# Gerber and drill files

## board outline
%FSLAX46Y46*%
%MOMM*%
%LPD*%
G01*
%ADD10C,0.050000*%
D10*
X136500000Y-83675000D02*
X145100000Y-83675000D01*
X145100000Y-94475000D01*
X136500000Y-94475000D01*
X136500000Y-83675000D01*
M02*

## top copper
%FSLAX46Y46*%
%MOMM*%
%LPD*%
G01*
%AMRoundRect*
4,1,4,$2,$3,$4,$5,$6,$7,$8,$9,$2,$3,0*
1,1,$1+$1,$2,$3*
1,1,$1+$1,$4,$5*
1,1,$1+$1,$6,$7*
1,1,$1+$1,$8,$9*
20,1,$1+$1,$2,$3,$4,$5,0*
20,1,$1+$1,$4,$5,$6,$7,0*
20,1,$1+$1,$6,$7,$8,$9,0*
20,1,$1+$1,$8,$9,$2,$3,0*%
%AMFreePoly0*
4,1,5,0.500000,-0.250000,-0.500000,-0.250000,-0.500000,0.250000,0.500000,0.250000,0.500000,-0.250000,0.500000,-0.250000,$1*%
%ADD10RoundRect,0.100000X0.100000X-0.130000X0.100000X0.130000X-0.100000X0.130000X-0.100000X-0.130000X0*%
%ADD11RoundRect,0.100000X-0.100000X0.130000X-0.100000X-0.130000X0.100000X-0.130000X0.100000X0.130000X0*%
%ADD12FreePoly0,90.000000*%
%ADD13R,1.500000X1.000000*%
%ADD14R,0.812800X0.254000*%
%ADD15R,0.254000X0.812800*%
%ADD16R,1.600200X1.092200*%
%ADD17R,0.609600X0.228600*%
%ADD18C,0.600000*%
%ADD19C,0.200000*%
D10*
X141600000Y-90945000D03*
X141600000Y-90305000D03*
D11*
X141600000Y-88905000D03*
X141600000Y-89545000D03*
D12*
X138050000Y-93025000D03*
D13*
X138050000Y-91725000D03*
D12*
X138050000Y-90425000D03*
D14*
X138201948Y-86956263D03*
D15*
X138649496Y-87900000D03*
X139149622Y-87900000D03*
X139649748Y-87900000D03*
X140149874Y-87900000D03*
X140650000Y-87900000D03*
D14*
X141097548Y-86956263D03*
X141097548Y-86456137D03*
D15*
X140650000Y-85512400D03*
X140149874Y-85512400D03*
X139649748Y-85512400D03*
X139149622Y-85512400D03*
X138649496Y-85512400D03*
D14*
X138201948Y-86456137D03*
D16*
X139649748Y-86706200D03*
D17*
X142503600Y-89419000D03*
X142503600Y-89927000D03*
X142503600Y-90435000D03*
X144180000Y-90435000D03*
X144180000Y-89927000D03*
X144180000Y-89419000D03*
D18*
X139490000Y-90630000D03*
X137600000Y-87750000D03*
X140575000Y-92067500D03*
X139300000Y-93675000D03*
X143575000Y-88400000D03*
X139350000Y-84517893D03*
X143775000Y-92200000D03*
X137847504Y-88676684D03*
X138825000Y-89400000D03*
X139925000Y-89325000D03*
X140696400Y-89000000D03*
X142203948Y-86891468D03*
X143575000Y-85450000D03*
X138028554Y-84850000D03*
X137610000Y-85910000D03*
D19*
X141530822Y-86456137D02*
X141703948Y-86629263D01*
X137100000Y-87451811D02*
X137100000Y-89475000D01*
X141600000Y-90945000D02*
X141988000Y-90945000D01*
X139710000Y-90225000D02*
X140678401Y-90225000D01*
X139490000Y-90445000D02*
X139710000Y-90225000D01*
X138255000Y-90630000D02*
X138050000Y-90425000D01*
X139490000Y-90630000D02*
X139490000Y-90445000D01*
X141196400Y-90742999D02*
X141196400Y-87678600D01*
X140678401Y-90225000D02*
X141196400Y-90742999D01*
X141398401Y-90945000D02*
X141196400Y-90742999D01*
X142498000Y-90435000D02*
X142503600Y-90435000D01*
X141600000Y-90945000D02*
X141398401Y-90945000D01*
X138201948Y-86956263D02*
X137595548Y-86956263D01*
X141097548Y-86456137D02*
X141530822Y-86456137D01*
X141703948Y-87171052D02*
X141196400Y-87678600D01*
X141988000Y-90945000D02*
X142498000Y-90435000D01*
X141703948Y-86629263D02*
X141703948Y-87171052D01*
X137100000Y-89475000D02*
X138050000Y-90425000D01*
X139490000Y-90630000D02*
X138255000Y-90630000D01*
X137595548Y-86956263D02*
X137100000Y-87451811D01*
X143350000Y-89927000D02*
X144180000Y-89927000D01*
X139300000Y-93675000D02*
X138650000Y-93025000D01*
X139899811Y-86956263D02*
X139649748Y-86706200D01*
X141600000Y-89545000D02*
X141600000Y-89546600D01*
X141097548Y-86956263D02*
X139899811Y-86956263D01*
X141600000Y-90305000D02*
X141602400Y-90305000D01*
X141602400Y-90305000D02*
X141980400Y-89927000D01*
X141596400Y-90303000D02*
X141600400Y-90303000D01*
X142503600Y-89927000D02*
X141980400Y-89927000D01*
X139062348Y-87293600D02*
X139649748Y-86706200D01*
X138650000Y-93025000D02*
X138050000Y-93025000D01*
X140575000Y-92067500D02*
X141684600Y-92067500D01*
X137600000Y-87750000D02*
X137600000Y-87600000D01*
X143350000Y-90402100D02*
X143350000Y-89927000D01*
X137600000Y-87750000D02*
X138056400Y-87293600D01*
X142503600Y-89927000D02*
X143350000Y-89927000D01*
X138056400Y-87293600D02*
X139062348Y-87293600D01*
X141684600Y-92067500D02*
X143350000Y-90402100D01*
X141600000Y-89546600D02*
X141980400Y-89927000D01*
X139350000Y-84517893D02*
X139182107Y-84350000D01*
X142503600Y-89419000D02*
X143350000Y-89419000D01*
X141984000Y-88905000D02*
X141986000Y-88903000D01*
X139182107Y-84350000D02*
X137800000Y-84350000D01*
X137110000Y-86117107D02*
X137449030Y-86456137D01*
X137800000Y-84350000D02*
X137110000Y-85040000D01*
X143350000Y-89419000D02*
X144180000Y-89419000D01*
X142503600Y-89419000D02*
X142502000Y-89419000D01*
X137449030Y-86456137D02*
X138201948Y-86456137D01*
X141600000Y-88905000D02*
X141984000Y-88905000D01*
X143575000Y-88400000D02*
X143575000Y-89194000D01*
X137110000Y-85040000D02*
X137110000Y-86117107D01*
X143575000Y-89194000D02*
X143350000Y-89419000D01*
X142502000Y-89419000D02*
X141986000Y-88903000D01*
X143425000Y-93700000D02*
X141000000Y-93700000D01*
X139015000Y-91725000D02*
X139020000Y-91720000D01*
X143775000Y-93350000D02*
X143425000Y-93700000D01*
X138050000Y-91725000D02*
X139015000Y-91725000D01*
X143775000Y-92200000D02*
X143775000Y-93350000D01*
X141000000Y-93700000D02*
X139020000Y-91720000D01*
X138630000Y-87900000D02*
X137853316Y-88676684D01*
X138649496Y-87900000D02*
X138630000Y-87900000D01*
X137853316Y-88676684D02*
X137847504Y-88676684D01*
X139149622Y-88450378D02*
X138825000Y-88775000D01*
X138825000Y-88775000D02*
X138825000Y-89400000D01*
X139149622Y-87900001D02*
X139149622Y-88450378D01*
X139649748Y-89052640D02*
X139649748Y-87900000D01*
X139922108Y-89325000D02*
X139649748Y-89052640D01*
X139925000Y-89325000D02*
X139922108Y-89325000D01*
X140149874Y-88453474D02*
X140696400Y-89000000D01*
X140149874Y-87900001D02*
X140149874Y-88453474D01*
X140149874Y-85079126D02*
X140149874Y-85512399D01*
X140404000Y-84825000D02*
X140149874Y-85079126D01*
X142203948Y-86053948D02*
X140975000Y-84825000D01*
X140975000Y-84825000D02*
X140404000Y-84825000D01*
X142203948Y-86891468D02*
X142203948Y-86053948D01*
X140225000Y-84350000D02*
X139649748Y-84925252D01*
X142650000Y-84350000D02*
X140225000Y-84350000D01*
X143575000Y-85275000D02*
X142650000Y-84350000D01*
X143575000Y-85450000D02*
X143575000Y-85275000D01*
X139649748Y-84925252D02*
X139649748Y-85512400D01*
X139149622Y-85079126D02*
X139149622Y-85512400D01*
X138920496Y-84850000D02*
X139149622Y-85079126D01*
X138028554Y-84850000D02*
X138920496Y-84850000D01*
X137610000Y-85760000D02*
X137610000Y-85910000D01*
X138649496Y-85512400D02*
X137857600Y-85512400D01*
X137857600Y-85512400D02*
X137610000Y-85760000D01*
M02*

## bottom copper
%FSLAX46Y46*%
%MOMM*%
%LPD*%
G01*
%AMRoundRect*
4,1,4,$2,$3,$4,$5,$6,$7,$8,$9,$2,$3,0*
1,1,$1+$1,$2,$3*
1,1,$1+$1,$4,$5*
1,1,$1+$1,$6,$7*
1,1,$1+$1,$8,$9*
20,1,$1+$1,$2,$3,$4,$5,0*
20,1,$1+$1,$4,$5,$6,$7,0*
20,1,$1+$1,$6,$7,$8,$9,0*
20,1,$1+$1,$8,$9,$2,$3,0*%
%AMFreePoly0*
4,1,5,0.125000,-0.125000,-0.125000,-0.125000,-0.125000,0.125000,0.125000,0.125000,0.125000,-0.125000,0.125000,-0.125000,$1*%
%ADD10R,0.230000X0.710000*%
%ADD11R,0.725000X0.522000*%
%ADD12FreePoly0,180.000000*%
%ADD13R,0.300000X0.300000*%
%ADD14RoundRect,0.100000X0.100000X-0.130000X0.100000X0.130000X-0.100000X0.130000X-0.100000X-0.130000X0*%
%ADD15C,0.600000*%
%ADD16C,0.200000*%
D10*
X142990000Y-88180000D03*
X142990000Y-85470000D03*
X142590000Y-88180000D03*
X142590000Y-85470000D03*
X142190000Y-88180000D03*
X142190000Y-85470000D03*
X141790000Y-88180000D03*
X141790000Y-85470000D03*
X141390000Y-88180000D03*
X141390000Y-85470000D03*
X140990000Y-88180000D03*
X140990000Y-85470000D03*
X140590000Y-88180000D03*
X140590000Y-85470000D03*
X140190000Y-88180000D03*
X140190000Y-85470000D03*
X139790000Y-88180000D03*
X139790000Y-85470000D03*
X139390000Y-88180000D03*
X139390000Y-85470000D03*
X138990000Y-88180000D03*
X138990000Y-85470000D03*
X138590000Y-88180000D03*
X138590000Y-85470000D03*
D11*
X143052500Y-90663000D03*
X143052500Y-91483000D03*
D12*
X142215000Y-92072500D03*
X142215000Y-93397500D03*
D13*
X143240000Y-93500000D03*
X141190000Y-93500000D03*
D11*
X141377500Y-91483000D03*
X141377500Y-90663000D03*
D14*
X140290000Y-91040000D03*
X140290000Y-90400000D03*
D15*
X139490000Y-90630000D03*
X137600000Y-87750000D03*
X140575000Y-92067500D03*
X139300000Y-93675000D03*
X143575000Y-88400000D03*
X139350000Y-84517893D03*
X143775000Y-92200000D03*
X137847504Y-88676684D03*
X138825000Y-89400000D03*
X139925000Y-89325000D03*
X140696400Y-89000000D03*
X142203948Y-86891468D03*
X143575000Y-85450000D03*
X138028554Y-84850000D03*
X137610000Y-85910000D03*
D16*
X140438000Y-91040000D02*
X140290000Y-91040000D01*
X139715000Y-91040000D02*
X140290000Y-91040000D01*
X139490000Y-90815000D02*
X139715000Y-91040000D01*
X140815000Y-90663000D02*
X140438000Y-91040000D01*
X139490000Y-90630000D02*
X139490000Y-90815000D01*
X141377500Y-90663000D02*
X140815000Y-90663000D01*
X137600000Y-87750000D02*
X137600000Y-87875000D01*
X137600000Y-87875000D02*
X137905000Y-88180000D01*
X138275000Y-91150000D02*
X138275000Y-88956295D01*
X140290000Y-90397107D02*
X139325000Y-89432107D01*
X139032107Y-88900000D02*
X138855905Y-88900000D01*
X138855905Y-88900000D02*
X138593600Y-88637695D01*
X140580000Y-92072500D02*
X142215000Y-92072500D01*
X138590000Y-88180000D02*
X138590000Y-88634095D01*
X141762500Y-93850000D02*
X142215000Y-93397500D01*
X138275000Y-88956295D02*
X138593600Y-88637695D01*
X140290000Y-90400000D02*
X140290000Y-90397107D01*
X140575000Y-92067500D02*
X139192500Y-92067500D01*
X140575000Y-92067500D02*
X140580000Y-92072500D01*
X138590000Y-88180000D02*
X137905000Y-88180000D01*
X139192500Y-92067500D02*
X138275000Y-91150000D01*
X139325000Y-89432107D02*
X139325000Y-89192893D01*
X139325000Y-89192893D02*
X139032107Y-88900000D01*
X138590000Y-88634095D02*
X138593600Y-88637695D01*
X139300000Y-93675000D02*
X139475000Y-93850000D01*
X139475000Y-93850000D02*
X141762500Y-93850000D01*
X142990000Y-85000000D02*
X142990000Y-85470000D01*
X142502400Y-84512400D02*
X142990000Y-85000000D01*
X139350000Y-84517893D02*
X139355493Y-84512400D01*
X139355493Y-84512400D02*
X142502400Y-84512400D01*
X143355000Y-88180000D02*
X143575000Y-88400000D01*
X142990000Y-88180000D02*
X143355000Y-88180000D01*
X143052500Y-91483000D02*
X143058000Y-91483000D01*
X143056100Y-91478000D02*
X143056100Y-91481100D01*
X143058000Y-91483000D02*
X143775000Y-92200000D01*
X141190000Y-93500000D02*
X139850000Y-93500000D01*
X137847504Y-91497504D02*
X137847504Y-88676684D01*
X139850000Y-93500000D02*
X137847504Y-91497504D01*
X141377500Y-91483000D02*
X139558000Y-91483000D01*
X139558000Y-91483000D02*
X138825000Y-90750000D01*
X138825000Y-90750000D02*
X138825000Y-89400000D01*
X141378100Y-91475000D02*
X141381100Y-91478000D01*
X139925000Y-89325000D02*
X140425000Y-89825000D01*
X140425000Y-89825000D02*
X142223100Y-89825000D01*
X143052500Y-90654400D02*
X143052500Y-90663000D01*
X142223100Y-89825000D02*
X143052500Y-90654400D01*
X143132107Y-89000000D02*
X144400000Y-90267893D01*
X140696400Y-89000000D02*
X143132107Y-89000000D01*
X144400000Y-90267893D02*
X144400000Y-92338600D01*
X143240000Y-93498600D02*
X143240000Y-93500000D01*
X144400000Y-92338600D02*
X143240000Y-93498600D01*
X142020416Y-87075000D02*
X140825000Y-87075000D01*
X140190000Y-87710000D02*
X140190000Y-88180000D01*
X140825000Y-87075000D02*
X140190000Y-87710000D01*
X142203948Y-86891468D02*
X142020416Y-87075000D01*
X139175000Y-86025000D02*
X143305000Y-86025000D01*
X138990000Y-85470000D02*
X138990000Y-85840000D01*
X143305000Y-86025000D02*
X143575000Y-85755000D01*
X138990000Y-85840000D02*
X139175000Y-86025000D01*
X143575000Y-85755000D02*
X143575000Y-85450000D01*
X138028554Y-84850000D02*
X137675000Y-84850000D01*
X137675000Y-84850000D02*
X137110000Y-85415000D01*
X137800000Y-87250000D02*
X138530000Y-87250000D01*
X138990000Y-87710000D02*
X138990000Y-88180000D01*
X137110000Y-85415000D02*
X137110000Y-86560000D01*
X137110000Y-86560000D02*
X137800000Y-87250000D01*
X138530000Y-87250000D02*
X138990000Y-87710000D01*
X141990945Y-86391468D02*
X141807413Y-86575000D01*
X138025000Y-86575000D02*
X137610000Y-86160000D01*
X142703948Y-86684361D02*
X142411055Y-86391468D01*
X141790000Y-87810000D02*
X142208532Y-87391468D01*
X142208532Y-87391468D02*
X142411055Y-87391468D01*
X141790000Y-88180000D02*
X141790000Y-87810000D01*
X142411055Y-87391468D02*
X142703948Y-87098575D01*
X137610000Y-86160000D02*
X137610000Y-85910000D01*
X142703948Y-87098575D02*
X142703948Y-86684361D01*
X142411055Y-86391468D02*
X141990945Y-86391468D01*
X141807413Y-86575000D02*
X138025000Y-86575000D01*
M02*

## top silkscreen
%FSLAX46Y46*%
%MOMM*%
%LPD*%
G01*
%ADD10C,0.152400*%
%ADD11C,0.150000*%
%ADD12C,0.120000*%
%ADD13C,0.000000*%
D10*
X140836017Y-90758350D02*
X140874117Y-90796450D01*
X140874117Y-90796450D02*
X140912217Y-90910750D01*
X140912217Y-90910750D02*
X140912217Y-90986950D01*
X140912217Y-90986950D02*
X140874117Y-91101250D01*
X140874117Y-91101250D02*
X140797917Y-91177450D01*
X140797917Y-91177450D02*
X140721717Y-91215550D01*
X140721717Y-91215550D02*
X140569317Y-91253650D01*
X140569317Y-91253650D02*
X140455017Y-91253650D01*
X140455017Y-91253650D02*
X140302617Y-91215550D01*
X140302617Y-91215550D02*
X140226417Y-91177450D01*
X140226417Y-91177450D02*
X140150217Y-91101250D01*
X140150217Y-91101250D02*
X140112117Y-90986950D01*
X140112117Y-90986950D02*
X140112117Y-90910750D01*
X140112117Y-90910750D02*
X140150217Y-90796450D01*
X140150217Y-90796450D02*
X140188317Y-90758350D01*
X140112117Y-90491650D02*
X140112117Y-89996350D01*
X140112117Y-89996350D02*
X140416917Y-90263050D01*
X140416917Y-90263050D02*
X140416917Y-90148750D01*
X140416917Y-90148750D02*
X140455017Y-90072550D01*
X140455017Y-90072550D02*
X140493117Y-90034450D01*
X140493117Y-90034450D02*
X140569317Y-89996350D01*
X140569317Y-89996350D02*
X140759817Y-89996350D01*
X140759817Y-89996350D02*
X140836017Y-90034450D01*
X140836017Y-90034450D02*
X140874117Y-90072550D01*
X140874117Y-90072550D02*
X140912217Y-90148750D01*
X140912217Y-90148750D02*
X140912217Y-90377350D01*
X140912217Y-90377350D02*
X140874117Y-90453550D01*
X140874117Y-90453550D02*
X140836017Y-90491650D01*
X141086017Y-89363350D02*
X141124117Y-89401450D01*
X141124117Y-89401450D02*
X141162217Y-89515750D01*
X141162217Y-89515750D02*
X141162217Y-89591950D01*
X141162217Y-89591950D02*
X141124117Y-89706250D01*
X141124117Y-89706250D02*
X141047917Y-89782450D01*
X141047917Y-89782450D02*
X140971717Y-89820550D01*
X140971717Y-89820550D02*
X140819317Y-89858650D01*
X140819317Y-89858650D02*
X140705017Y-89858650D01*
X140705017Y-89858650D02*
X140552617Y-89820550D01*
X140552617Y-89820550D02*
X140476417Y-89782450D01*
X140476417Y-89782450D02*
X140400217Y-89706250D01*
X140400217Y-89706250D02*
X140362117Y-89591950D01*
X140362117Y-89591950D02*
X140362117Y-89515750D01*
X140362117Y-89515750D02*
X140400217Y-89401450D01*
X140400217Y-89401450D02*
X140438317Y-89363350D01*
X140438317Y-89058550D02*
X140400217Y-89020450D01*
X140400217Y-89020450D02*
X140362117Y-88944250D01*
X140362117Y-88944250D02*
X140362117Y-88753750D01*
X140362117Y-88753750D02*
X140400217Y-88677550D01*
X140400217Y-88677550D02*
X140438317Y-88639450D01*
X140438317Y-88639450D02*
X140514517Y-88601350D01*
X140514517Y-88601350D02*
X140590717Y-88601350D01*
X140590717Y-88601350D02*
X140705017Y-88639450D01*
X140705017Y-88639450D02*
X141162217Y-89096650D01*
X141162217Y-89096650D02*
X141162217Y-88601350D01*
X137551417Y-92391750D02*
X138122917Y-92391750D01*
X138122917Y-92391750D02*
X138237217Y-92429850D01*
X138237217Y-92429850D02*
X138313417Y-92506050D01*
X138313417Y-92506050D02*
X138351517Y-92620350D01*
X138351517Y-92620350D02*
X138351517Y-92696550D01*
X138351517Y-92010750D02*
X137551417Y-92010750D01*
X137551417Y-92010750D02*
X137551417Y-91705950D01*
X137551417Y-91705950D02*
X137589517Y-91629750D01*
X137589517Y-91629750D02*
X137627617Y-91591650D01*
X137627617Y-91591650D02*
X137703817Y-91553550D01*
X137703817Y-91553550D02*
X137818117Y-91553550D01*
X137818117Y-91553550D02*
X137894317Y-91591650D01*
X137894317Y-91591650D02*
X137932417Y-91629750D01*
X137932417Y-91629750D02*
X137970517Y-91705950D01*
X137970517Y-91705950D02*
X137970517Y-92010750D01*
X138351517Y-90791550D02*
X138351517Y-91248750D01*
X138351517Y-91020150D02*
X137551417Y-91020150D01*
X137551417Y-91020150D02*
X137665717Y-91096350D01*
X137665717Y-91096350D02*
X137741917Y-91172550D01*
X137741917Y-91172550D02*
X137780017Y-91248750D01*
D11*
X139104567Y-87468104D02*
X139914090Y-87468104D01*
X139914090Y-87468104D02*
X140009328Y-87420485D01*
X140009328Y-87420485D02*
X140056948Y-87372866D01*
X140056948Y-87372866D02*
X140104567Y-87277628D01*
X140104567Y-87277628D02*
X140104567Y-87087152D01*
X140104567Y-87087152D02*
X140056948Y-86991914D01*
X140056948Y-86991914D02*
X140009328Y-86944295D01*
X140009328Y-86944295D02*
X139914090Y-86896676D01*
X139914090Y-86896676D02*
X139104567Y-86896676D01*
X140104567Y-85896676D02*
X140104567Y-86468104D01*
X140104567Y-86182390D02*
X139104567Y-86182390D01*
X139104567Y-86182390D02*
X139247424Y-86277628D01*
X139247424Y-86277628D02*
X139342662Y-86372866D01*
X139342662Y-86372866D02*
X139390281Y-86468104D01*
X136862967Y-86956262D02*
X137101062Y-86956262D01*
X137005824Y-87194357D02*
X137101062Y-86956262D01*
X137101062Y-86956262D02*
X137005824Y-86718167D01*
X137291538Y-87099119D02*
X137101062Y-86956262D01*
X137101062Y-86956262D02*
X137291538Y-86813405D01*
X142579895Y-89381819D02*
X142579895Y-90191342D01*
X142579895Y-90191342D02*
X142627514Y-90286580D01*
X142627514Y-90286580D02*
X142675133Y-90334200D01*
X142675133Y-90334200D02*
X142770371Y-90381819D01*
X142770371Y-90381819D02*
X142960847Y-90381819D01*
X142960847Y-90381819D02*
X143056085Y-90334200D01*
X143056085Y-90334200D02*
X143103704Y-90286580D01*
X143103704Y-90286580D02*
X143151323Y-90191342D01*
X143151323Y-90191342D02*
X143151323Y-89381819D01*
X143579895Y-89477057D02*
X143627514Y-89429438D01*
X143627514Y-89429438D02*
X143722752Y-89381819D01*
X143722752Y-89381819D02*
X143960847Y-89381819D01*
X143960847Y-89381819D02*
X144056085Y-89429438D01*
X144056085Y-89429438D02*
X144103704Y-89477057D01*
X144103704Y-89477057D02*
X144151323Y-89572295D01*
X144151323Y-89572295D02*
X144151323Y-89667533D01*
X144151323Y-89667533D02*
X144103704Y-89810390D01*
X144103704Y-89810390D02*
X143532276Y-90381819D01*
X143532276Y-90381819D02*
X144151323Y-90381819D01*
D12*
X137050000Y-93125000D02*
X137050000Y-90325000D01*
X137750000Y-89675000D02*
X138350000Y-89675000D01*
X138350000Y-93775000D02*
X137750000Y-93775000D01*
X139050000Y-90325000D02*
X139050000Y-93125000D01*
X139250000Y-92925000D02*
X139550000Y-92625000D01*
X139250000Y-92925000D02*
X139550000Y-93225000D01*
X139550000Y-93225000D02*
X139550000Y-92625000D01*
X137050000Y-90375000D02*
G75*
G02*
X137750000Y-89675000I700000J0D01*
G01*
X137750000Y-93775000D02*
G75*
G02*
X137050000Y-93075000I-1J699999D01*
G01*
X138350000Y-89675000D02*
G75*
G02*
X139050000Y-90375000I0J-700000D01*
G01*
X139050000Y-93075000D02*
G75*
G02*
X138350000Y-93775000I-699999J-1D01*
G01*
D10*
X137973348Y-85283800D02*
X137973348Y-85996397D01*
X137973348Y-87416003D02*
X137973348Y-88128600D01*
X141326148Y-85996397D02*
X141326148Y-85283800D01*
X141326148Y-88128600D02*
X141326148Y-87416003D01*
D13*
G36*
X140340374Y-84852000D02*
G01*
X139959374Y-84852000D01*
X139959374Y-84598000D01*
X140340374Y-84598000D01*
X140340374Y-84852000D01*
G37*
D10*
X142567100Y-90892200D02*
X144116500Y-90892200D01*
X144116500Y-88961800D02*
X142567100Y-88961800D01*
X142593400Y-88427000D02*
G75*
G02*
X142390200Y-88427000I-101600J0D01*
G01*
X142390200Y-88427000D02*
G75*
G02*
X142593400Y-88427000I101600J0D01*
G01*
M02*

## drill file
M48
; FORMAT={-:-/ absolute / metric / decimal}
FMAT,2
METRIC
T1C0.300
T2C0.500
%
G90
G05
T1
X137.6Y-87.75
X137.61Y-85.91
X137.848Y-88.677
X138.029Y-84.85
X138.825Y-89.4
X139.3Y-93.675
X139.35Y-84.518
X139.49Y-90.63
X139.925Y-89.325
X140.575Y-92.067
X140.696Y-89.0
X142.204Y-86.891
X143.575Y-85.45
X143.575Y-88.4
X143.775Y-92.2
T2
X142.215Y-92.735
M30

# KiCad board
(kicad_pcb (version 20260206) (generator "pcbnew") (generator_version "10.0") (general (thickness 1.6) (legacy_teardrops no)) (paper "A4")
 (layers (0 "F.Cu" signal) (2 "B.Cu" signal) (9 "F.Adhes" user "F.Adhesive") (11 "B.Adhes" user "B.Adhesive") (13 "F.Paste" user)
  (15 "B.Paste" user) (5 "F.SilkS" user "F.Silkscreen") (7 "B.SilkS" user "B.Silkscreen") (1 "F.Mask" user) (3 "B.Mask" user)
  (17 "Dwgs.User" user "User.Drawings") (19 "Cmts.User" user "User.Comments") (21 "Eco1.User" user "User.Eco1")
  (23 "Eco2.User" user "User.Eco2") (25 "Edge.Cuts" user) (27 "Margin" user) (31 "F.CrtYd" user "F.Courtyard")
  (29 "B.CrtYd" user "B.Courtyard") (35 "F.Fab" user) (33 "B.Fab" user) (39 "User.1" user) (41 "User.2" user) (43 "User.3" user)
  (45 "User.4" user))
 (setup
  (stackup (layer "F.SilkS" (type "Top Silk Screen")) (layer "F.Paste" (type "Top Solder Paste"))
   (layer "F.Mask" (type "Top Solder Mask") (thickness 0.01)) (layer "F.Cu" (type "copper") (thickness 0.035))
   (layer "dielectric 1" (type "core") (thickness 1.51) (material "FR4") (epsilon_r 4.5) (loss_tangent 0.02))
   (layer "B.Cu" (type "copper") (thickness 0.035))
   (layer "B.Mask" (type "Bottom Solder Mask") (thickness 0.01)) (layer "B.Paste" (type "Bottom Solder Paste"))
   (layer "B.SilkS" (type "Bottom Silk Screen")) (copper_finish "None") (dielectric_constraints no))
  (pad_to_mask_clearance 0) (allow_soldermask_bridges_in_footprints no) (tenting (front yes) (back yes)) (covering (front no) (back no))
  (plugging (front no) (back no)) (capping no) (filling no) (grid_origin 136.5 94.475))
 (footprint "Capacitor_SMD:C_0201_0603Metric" (layer "F.Cu") (at 141.6 90.625 90)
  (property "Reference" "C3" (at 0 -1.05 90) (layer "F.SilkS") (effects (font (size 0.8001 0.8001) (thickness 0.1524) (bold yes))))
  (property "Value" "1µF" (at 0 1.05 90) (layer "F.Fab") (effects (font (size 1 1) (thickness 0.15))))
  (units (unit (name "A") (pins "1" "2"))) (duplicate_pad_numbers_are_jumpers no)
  (pad "" smd roundrect (at -0.345 0 90) (size 0.318 0.36) (layers "F.Paste") (roundrect_rratio 0.25))
  (pad "" smd roundrect (at 0.345 0 90) (size 0.318 0.36) (layers "F.Paste") (roundrect_rratio 0.25))
  (pad "1" smd roundrect (at -0.32 0 90) (size 0.46 0.4) (layers "F.Cu" "F.Mask") (roundrect_rratio 0.25) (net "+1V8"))
  (pad "2" smd roundrect (at 0.32 0 90) (size 0.46 0.4) (layers "F.Cu" "F.Mask") (roundrect_rratio 0.25) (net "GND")))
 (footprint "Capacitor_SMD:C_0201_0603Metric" (layer "F.Cu") (at 141.6 89.225 -90)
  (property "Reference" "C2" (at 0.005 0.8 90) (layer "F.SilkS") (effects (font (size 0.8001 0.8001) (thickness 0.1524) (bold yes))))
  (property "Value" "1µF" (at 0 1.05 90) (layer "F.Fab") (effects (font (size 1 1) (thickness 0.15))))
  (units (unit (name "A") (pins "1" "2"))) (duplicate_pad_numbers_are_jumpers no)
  (pad "" smd roundrect (at -0.345 0 270) (size 0.318 0.36) (layers "F.Paste") (roundrect_rratio 0.25))
  (pad "" smd roundrect (at 0.345 0 270) (size 0.318 0.36) (layers "F.Paste") (roundrect_rratio 0.25))
  (pad "1" smd roundrect (at -0.32 0 270) (size 0.46 0.4) (layers "F.Cu" "F.Mask") (roundrect_rratio 0.25) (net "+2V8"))
  (pad "2" smd roundrect (at 0.32 0 270) (size 0.46 0.4) (layers "F.Cu" "F.Mask") (roundrect_rratio 0.25) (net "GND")))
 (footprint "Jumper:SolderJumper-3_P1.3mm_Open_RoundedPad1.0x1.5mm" (layer "F.Cu") (at 138.05 91.725 90)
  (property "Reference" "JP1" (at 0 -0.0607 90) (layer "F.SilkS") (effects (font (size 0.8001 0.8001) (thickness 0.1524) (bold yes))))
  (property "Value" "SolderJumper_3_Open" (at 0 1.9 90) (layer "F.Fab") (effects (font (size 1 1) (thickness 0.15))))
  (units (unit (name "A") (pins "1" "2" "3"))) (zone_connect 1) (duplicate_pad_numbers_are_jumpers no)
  (fp_line (start -1.4 -1) (end 1.4 -1) (stroke (width 0.12) (type solid)) (layer "F.SilkS"))
  (fp_line (start 2.05 -0.3) (end 2.05 0.3) (stroke (width 0.12) (type solid)) (layer "F.SilkS"))
  (fp_line (start -2.05 0.3) (end -2.05 -0.3) (stroke (width 0.12) (type solid)) (layer "F.SilkS"))
  (fp_line (start 1.4 1) (end -1.4 1) (stroke (width 0.12) (type solid)) (layer "F.SilkS"))
  (fp_line (start -1.2 1.2) (end -0.9 1.5) (stroke (width 0.12) (type solid)) (layer "F.SilkS"))
  (fp_line (start -1.2 1.2) (end -1.5 1.5) (stroke (width 0.12) (type solid)) (layer "F.SilkS"))
  (fp_line (start -1.5 1.5) (end -0.9 1.5) (stroke (width 0.12) (type solid)) (layer "F.SilkS"))
  (fp_arc (start 1.35 -1) (mid 1.844975 -0.794975) (end 2.05 -0.3) (stroke (width 0.12) (type solid)) (layer "F.SilkS"))
  (fp_arc (start -2.05 -0.3) (mid -1.844975 -0.794975) (end -1.35 -1) (stroke (width 0.12) (type solid)) (layer "F.SilkS"))
  (fp_arc (start 2.05 0.3) (mid 1.844975 0.794975) (end 1.35 1) (stroke (width 0.12) (type solid)) (layer "F.SilkS"))
  (fp_arc (start -1.35 1) (mid -1.844975 0.794975) (end -2.05 0.3) (stroke (width 0.12) (type solid)) (layer "F.SilkS"))
  (pad "1" smd custom (at -1.3 0 90) (size 1 0.5) (layers "F.Cu" "F.Mask") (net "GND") (zone_connect 2) (thermal_bridge_angle 45)
   (options (clearance outline) (anchor rect)) (primitives))
  (pad "2" smd rect (at 0 0 90) (size 1 1.5) (layers "F.Cu" "F.Mask") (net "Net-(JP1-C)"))
  (pad "3" smd custom (at 1.3 0 90) (size 1 0.5) (layers "F.Cu" "F.Mask") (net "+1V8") (zone_connect 2) (thermal_bridge_angle 45)
   (options (clearance outline) (anchor rect)) (primitives)))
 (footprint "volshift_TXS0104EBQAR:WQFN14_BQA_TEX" (layer "F.Cu") (at 139.649748 86.7062 90)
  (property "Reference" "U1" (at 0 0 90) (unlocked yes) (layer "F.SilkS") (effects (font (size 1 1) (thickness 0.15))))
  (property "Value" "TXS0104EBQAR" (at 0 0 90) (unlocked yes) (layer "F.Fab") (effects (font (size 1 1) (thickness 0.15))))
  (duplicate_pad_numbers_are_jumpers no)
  (fp_line (start 1.4224 -1.6764) (end 0.709803 -1.6764) (stroke (width 0.1524) (type solid)) (layer "F.SilkS"))
  (fp_line (start -0.709803 -1.6764) (end -1.4224 -1.6764) (stroke (width 0.1524) (type solid)) (layer "F.SilkS"))
  (fp_line (start 0.709803 1.6764) (end 1.4224 1.6764) (stroke (width 0.1524) (type solid)) (layer "F.SilkS"))
  (fp_line (start -1.4224 1.6764) (end -0.709803 1.6764) (stroke (width 0.1524) (type solid)) (layer "F.SilkS"))
  (fp_poly
   (pts (xy 2.1082 0.309626) (xy 2.1082 0.690626) (xy 1.8542 0.690626) (xy 1.8542 0.309626)) (stroke (width 0) (type solid)) (fill yes)
   (layer "F.SilkS"))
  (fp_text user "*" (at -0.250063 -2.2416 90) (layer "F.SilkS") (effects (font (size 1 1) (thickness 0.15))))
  (pad "1" smd rect (at -0.250063 -1.4478 90) (size 0.254 0.8128) (layers "F.Cu" "F.Mask" "F.Paste") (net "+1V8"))
  (pad "2" smd rect (at -1.1938 -1.000252 180) (size 0.254 0.8128) (layers "F.Cu" "F.Mask" "F.Paste") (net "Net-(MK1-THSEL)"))
  (pad "3" smd rect (at -1.1938 -0.500126 180) (size 0.254 0.8128) (layers "F.Cu" "F.Mask" "F.Paste") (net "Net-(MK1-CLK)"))
  (pad "4" smd rect (at -1.1938 0 180) (size 0.254 0.8128) (layers "F.Cu" "F.Mask" "F.Paste") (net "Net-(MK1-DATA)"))
  (pad "5" smd rect (at -1.1938 0.500126 180) (size 0.254 0.8128) (layers "F.Cu" "F.Mask" "F.Paste") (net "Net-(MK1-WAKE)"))
  (pad "6" smd rect (at -1.1938 1.000252 180) (size 0.254 0.8128) (layers "F.Cu" "F.Mask" "F.Paste") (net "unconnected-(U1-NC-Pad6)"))
  (pad "7" smd rect (at -0.250063 1.4478 90) (size 0.254 0.8128) (layers "F.Cu" "F.Mask" "F.Paste") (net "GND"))
  (pad "8" smd rect (at 0.250063 1.4478 90) (size 0.254 0.8128) (layers "F.Cu" "F.Mask" "F.Paste") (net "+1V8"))
  (pad "9" smd rect (at 1.1938 1.000252 180) (size 0.254 0.8128) (layers "F.Cu" "F.Mask" "F.Paste") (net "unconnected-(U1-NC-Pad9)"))
  (pad "10" smd rect (at 1.1938 0.500126 180) (size 0.254 0.8128) (layers "F.Cu" "F.Mask" "F.Paste") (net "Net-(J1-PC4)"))
  (pad "11" smd rect (at 1.1938 0 180) (size 0.254 0.8128) (layers "F.Cu" "F.Mask" "F.Paste") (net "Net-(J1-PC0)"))
  (pad "12" smd rect (at 1.1938 -0.500126 180) (size 0.254 0.8128) (layers "F.Cu" "F.Mask" "F.Paste") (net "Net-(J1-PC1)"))
  (pad "13" smd rect (at 1.1938 -1.000252 180) (size 0.254 0.8128) (layers "F.Cu" "F.Mask" "F.Paste") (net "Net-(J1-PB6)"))
  (pad "14" smd rect (at 0.250063 -1.4478 90) (size 0.254 0.8128) (layers "F.Cu" "F.Mask" "F.Paste") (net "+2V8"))
  (pad "15" smd rect (at 0 0 90) (size 1.0922 1.6002) (layers "F.Cu" "F.Mask" "F.Paste") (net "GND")))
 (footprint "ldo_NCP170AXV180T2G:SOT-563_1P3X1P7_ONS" (layer "F.Cu") (at 143.3418 89.927)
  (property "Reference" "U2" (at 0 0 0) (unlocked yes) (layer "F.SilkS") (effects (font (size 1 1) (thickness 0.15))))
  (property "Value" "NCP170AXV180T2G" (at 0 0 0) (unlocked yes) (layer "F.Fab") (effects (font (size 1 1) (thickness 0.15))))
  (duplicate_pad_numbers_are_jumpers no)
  (fp_line (start -0.7747 0.9652) (end 0.7747 0.9652) (stroke (width 0.1524) (type solid)) (layer "F.SilkS"))
  (fp_line (start 0.7747 -0.9652) (end -0.7747 -0.9652) (stroke (width 0.1524) (type solid)) (layer "F.SilkS"))
  (fp_circle (center -0.85 -1.5) (end -0.7484 -1.5) (stroke (width 0.1524) (type solid)) (fill no) (layer "F.SilkS"))
  (pad "1" smd rect (at -0.8382 -0.508) (size 0.6096 0.2286) (layers "F.Cu" "F.Mask" "F.Paste") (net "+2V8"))
  (pad "2" smd rect (at -0.8382 0) (size 0.6096 0.2286) (layers "F.Cu" "F.Mask" "F.Paste") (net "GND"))
  (pad "3" smd rect (at -0.8382 0.508) (size 0.6096 0.2286) (layers "F.Cu" "F.Mask" "F.Paste") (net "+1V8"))
  (pad "4" smd rect (at 0.8382 0.508) (size 0.6096 0.2286) (layers "F.Cu" "F.Mask" "F.Paste") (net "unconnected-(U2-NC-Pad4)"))
  (pad "5" smd rect (at 0.8382 0) (size 0.6096 0.2286) (layers "F.Cu" "F.Mask" "F.Paste") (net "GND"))
  (pad "6" smd rect (at 0.8382 -0.508) (size 0.6096 0.2286) (layers "F.Cu" "F.Mask" "F.Paste") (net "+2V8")))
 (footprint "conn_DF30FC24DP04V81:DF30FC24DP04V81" (layer "B.Cu") (at 140.79 86.825 180)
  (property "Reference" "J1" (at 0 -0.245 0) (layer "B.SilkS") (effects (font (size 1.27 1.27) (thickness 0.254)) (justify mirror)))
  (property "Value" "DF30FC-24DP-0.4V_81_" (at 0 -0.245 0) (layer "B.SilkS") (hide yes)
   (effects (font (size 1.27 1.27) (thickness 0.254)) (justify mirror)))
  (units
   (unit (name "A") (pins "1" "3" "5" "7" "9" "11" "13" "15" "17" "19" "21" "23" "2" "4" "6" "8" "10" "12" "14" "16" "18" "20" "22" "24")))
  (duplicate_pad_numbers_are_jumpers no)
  (pad "1" smd rect (at -2.2 -1.355 180) (size 0.23 0.71) (layers "B.Cu" "B.Mask" "B.Paste") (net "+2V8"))
  (pad "2" smd rect (at -2.2 1.355 180) (size 0.23 0.71) (layers "B.Cu" "B.Mask" "B.Paste") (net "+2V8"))
  (pad "3" smd rect (at -1.8 -1.355 180) (size 0.23 0.71) (layers "B.Cu" "B.Mask" "B.Paste") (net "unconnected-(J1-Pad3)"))
  (pad "4" smd rect (at -1.8 1.355 180) (size 0.23 0.71) (layers "B.Cu" "B.Mask" "B.Paste") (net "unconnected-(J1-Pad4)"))
  (pad "5" smd rect (at -1.4 -1.355 180) (size 0.23 0.71) (layers "B.Cu" "B.Mask" "B.Paste") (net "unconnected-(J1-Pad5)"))
  (pad "6" smd rect (at -1.4 1.355 180) (size 0.23 0.71) (layers "B.Cu" "B.Mask" "B.Paste") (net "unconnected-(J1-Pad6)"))
  (pad "7" smd rect (at -1 -1.355 180) (size 0.23 0.71) (layers "B.Cu" "B.Mask" "B.Paste") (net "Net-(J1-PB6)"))
  (pad "8" smd rect (at -1 1.355 180) (size 0.23 0.71) (layers "B.Cu" "B.Mask" "B.Paste") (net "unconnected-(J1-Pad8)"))
  (pad "9" smd rect (at -0.6 -1.355 180) (size 0.23 0.71) (layers "B.Cu" "B.Mask" "B.Paste") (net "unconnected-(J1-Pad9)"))
  (pad "10" smd rect (at -0.6 1.355 180) (size 0.23 0.71) (layers "B.Cu" "B.Mask" "B.Paste") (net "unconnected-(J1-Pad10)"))
  (pad "11" smd rect (at -0.2 -1.355 180) (size 0.23 0.71) (layers "B.Cu" "B.Mask" "B.Paste") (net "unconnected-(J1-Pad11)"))
  (pad "12" smd rect (at -0.2 1.355 180) (size 0.23 0.71) (layers "B.Cu" "B.Mask" "B.Paste") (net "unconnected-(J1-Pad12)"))
  (pad "13" smd rect (at 0.2 -1.355 180) (size 0.23 0.71) (layers "B.Cu" "B.Mask" "B.Paste") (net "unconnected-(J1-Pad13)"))
  (pad "14" smd rect (at 0.2 1.355 180) (size 0.23 0.71) (layers "B.Cu" "B.Mask" "B.Paste") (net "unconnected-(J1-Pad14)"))
  (pad "15" smd rect (at 0.6 -1.355 180) (size 0.23 0.71) (layers "B.Cu" "B.Mask" "B.Paste") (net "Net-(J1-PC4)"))
  (pad "16" smd rect (at 0.6 1.355 180) (size 0.23 0.71) (layers "B.Cu" "B.Mask" "B.Paste") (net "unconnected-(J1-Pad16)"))
  (pad "17" smd rect (at 1 -1.355 180) (size 0.23 0.71) (layers "B.Cu" "B.Mask" "B.Paste") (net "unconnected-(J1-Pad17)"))
  (pad "18" smd rect (at 1 1.355 180) (size 0.23 0.71) (layers "B.Cu" "B.Mask" "B.Paste") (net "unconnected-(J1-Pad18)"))
  (pad "19" smd rect (at 1.4 -1.355 180) (size 0.23 0.71) (layers "B.Cu" "B.Mask" "B.Paste") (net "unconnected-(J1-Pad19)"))
  (pad "20" smd rect (at 1.4 1.355 180) (size 0.23 0.71) (layers "B.Cu" "B.Mask" "B.Paste") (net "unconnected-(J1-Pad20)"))
  (pad "21" smd rect (at 1.8 -1.355 180) (size 0.23 0.71) (layers "B.Cu" "B.Mask" "B.Paste") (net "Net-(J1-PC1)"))
  (pad "22" smd rect (at 1.8 1.355 180) (size 0.23 0.71) (layers "B.Cu" "B.Mask" "B.Paste") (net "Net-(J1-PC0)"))
  (pad "23" smd rect (at 2.2 -1.355 180) (size 0.23 0.71) (layers "B.Cu" "B.Mask" "B.Paste") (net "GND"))
  (pad "24" smd rect (at 2.2 1.355 180) (size 0.23 0.71) (layers "B.Cu" "B.Mask" "B.Paste") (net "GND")))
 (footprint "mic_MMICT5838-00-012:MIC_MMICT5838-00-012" (layer "B.Cu") (at 142.215 92.025 180)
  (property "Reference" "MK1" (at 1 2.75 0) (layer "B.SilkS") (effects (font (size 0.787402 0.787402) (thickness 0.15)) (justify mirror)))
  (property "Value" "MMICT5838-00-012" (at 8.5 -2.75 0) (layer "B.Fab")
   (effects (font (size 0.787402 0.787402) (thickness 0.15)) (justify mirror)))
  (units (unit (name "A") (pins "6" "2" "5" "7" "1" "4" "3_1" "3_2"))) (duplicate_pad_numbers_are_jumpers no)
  (pad "" np_thru_hole circle (at 0 -0.71 180) (size 0.5 0.5) (drill 0.5) (layers "*.Cu" "*.Mask"))
  (pad "1" smd rect (at -0.8375 1.362 180) (size 0.725 0.522) (layers "B.Cu") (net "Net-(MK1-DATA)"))
  (pad "2" smd rect (at -0.8375 0.542 180) (size 0.725 0.522) (layers "B.Cu") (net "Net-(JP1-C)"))
  (pad "3_1" smd custom (at 0 -0.0475 180) (size 0.25 0.25) (layers "B.Cu") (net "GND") (options (clearance outline) (anchor rect))
   (primitives))
  (pad "3_2" smd custom (at 0 -1.3725 180) (size 0.25 0.25) (layers "B.Cu") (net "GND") (options (clearance outline) (anchor rect))
   (primitives))
  (pad "4" smd rect (at -1.025 -1.475 180) (size 0.3 0.3) (layers "B.Cu") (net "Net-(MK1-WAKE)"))
  (pad "5" smd rect (at 1.025 -1.475 180) (size 0.3 0.3) (layers "B.Cu") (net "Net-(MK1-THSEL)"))
  (pad "6" smd rect (at 0.8375 0.542 180) (size 0.725 0.522) (layers "B.Cu") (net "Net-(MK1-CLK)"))
  (pad "7" smd rect (at 0.8375 1.362 180) (size 0.725 0.522) (layers "B.Cu") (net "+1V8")))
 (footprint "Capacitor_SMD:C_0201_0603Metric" (layer "B.Cu") (at 140.29 90.72 90)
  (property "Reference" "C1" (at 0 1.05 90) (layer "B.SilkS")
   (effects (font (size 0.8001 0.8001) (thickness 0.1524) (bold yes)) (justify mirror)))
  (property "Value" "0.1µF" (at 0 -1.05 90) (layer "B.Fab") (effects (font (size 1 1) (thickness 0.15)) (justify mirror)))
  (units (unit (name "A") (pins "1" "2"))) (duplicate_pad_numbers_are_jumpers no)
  (pad "" smd roundrect (at -0.345 0 90) (size 0.318 0.36) (layers "B.Paste") (roundrect_rratio 0.25))
  (pad "" smd roundrect (at 0.345 0 90) (size 0.318 0.36) (layers "B.Paste") (roundrect_rratio 0.25))
  (pad "1" smd roundrect (at -0.32 0 90) (size 0.46 0.4) (layers "B.Cu" "B.Mask") (roundrect_rratio 0.25) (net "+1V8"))
  (pad "2" smd roundrect (at 0.32 0 90) (size 0.46 0.4) (layers "B.Cu" "B.Mask") (roundrect_rratio 0.25) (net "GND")))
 (gr_rect (start 136.5 83.675) (end 145.1 94.475) (stroke (width 0.05) (type default)) (fill no) (layer "Edge.Cuts"))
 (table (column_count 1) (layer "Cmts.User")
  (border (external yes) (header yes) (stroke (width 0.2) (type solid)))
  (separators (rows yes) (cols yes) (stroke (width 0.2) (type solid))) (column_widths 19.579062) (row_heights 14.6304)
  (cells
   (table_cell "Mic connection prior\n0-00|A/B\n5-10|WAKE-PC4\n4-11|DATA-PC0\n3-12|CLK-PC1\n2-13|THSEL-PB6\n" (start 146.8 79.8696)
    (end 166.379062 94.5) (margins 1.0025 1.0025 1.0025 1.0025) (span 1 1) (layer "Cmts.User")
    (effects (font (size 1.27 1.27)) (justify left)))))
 (segment (start 141.530822 86.456137) (end 141.703948 86.629263) (width 0.2) (layer "F.Cu") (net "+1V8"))
 (segment (start 137.1 87.451811) (end 137.1 89.475) (width 0.2) (layer "F.Cu") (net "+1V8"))
 (segment (start 141.6 90.945) (end 141.988 90.945) (width 0.2) (layer "F.Cu") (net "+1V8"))
 (segment (start 139.71 90.225) (end 140.678401 90.225) (width 0.2) (layer "F.Cu") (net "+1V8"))
 (segment (start 139.49 90.445) (end 139.71 90.225) (width 0.2) (layer "F.Cu") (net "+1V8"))
 (segment (start 138.255 90.63) (end 138.05 90.425) (width 0.2) (layer "F.Cu") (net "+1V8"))
 (segment (start 139.49 90.63) (end 139.49 90.445) (width 0.2) (layer "F.Cu") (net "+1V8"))
 (segment (start 141.1964 90.742999) (end 141.1964 87.6786) (width 0.2) (layer "F.Cu") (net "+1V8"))
 (segment (start 140.678401 90.225) (end 141.1964 90.742999) (width 0.2) (layer "F.Cu") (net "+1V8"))
 (segment (start 141.398401 90.945) (end 141.1964 90.742999) (width 0.2) (layer "F.Cu") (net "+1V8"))
 (segment (start 142.498 90.435) (end 142.5036 90.435) (width 0.2) (layer "F.Cu") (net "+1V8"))
 (segment (start 141.6 90.945) (end 141.398401 90.945) (width 0.2) (layer "F.Cu") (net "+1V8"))
 (segment (start 138.201948 86.956263) (end 137.595548 86.956263) (width 0.2) (layer "F.Cu") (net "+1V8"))
 (segment (start 141.097548 86.456137) (end 141.530822 86.456137) (width 0.2) (layer "F.Cu") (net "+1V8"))
 (segment (start 141.703948 87.171052) (end 141.1964 87.6786) (width 0.2) (layer "F.Cu") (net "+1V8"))
 (segment (start 141.988 90.945) (end 142.498 90.435) (width 0.2) (layer "F.Cu") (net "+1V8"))
 (segment (start 141.703948 86.629263) (end 141.703948 87.171052) (width 0.2) (layer "F.Cu") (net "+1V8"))
 (segment (start 137.1 89.475) (end 138.05 90.425) (width 0.2) (layer "F.Cu") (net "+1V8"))
 (segment (start 139.49 90.63) (end 138.255 90.63) (width 0.2) (layer "F.Cu") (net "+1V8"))
 (segment (start 137.595548 86.956263) (end 137.1 87.451811) (width 0.2) (layer "F.Cu") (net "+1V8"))
 (via (at 139.49 90.63) (size 0.6) (drill 0.3) (layers "F.Cu" "B.Cu") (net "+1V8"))
 (segment (start 140.438 91.04) (end 140.29 91.04) (width 0.2) (layer "B.Cu") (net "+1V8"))
 (segment (start 139.715 91.04) (end 140.29 91.04) (width 0.2) (layer "B.Cu") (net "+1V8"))
 (segment (start 139.49 90.815) (end 139.715 91.04) (width 0.2) (layer "B.Cu") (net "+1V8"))
 (segment (start 140.815 90.663) (end 140.438 91.04) (width 0.2) (layer "B.Cu") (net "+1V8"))
 (segment (start 139.49 90.63) (end 139.49 90.815) (width 0.2) (layer "B.Cu") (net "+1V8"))
 (segment (start 141.3775 90.663) (end 140.815 90.663) (width 0.2) (layer "B.Cu") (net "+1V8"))
 (segment (start 143.35 89.927) (end 144.18 89.927) (width 0.2) (layer "F.Cu") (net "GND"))
 (segment (start 139.3 93.675) (end 138.65 93.025) (width 0.2) (layer "F.Cu") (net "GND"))
 (segment (start 139.899811 86.956263) (end 139.649748 86.7062) (width 0.2) (layer "F.Cu") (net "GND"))
 (segment (start 141.6 89.545) (end 141.6 89.5466) (width 0.2) (layer "F.Cu") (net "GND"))
 (segment (start 141.097548 86.956263) (end 139.899811 86.956263) (width 0.2) (layer "F.Cu") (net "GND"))
 (segment (start 141.6 90.305) (end 141.6024 90.305) (width 0.2) (layer "F.Cu") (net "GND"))
 (segment (start 141.6024 90.305) (end 141.9804 89.927) (width 0.2) (layer "F.Cu") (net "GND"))
 (segment (start 141.5964 90.303) (end 141.6004 90.303) (width 0.2) (layer "F.Cu") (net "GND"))
 (segment (start 142.5036 89.927) (end 141.9804 89.927) (width 0.2) (layer "F.Cu") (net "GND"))
 (segment (start 139.062348 87.2936) (end 139.649748 86.7062) (width 0.2) (layer "F.Cu") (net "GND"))
 (segment (start 138.65 93.025) (end 138.05 93.025) (width 0.2) (layer "F.Cu") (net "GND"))
 (segment (start 140.575 92.0675) (end 141.6846 92.0675) (width 0.2) (layer "F.Cu") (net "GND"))
 (segment (start 137.6 87.75) (end 137.6 87.6) (width 0.2) (layer "F.Cu") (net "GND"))
 (segment (start 143.35 90.4021) (end 143.35 89.927) (width 0.2) (layer "F.Cu") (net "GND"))
 (segment (start 137.6 87.75) (end 138.0564 87.2936) (width 0.2) (layer "F.Cu") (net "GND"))
 (segment (start 142.5036 89.927) (end 143.35 89.927) (width 0.2) (layer "F.Cu") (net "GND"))
 (segment (start 138.0564 87.2936) (end 139.062348 87.2936) (width 0.2) (layer "F.Cu") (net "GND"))
 (segment (start 141.6846 92.0675) (end 143.35 90.4021) (width 0.2) (layer "F.Cu") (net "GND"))
 (segment (start 141.6 89.5466) (end 141.9804 89.927) (width 0.2) (layer "F.Cu") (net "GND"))
 (via (at 137.6 87.75) (size 0.6) (drill 0.3) (layers "F.Cu" "B.Cu") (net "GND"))
 (via (at 140.575 92.0675) (size 0.6) (drill 0.3) (layers "F.Cu" "B.Cu") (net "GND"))
 (via (at 139.3 93.675) (size 0.6) (drill 0.3) (layers "F.Cu" "B.Cu") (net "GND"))
 (segment (start 137.6 87.75) (end 137.6 87.875) (width 0.2) (layer "B.Cu") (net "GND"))
 (segment (start 137.6 87.875) (end 137.905 88.18) (width 0.2) (layer "B.Cu") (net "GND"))
 (segment (start 138.275 91.15) (end 138.275 88.956295) (width 0.2) (layer "B.Cu") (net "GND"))
 (segment (start 140.29 90.397107) (end 139.325 89.432107) (width 0.2) (layer "B.Cu") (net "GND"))
 (segment (start 139.032107 88.9) (end 138.855905 88.9) (width 0.2) (layer "B.Cu") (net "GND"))
 (segment (start 138.855905 88.9) (end 138.5936 88.637695) (width 0.2) (layer "B.Cu") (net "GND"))
 (segment (start 140.58 92.0725) (end 142.215 92.0725) (width 0.2) (layer "B.Cu") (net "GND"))
 (segment (start 138.59 88.18) (end 138.59 88.634095) (width 0.2) (layer "B.Cu") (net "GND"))
 (segment (start 141.7625 93.85) (end 142.215 93.3975) (width 0.2) (layer "B.Cu") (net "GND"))
 (segment (start 138.275 88.956295) (end 138.5936 88.637695) (width 0.2) (layer "B.Cu") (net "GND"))
 (segment (start 140.29 90.4) (end 140.29 90.397107) (width 0.2) (layer "B.Cu") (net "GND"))
 (segment (start 140.575 92.0675) (end 139.1925 92.0675) (width 0.2) (layer "B.Cu") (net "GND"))
 (segment (start 140.575 92.0675) (end 140.58 92.0725) (width 0.2) (layer "B.Cu") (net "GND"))
 (segment (start 138.59 88.18) (end 137.905 88.18) (width 0.2) (layer "B.Cu") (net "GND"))
 (segment (start 139.1925 92.0675) (end 138.275 91.15) (width 0.2) (layer "B.Cu") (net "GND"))
 (segment (start 139.325 89.432107) (end 139.325 89.192893) (width 0.2) (layer "B.Cu") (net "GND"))
 (segment (start 139.325 89.192893) (end 139.032107 88.9) (width 0.2) (layer "B.Cu") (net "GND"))
 (segment (start 138.59 88.634095) (end 138.5936 88.637695) (width 0.2) (layer "B.Cu") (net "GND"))
 (segment (start 139.3 93.675) (end 139.475 93.85) (width 0.2) (layer "B.Cu") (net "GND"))
 (segment (start 139.475 93.85) (end 141.7625 93.85) (width 0.2) (layer "B.Cu") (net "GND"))
 (segment (start 139.35 84.517893) (end 139.182107 84.35) (width 0.2) (layer "F.Cu") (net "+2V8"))
 (segment (start 142.5036 89.419) (end 143.35 89.419) (width 0.2) (layer "F.Cu") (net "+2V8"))
 (segment (start 141.984 88.905) (end 141.986 88.903) (width 0.2) (layer "F.Cu") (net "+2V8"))
 (segment (start 139.182107 84.35) (end 137.8 84.35) (width 0.2) (layer "F.Cu") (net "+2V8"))
 (segment (start 137.11 86.117107) (end 137.44903 86.456137) (width 0.2) (layer "F.Cu") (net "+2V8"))
 (segment (start 137.8 84.35) (end 137.11 85.04) (width 0.2) (layer "F.Cu") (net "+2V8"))
 (segment (start 143.35 89.419) (end 144.18 89.419) (width 0.2) (layer "F.Cu") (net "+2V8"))
 (segment (start 142.5036 89.419) (end 142.502 89.419) (width 0.2) (layer "F.Cu") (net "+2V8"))
 (segment (start 137.44903 86.456137) (end 138.201948 86.456137) (width 0.2) (layer "F.Cu") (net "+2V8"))
 (segment (start 141.6 88.905) (end 141.984 88.905) (width 0.2) (layer "F.Cu") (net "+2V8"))
 (segment (start 143.575 88.4) (end 143.575 89.194) (width 0.2) (layer "F.Cu") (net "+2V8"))
 (segment (start 137.11 85.04) (end 137.11 86.117107) (width 0.2) (layer "F.Cu") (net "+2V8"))
 (segment (start 143.575 89.194) (end 143.35 89.419) (width 0.2) (layer "F.Cu") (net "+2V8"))
 (segment (start 142.502 89.419) (end 141.986 88.903) (width 0.2) (layer "F.Cu") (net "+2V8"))
 (via (at 143.575 88.4) (size 0.6) (drill 0.3) (layers "F.Cu" "B.Cu") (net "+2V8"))
 (via (at 139.35 84.517893) (size 0.6) (drill 0.3) (layers "F.Cu" "B.Cu") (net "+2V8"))
 (segment (start 142.99 85) (end 142.99 85.47) (width 0.2) (layer "B.Cu") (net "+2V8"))
 (segment (start 142.5024 84.5124) (end 142.99 85) (width 0.2) (layer "B.Cu") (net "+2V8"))
 (segment (start 139.35 84.517893) (end 139.355493 84.5124) (width 0.2) (layer "B.Cu") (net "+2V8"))
 (segment (start 139.355493 84.5124) (end 142.5024 84.5124) (width 0.2) (layer "B.Cu") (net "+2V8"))
 (segment (start 143.355 88.18) (end 143.575 88.4) (width 0.2) (layer "B.Cu") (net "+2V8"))
 (segment (start 142.99 88.18) (end 143.355 88.18) (width 0.2) (layer "B.Cu") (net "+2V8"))
 (segment (start 143.425 93.7) (end 141 93.7) (width 0.2) (layer "F.Cu") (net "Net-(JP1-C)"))
 (segment (start 139.015 91.725) (end 139.02 91.72) (width 0.2) (layer "F.Cu") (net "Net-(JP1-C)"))
 (segment (start 143.775 93.35) (end 143.425 93.7) (width 0.2) (layer "F.Cu") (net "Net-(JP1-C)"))
 (segment (start 138.05 91.725) (end 139.015 91.725) (width 0.2) (layer "F.Cu") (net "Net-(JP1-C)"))
 (segment (start 143.775 92.2) (end 143.775 93.35) (width 0.2) (layer "F.Cu") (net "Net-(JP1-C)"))
 (segment (start 141 93.7) (end 139.02 91.72) (width 0.2) (layer "F.Cu") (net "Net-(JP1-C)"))
 (via (at 143.775 92.2) (size 0.6) (drill 0.3) (layers "F.Cu" "B.Cu") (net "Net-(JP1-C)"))
 (segment (start 143.0525 91.483) (end 143.058 91.483) (width 0.2) (layer "B.Cu") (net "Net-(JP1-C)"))
 (segment (start 143.0561 91.478) (end 143.0561 91.4811) (width 0.2) (layer "B.Cu") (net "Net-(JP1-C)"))
 (segment (start 143.058 91.483) (end 143.775 92.2) (width 0.2) (layer "B.Cu") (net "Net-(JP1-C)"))
 (segment (start 138.63 87.9) (end 137.853316 88.676684) (width 0.2) (layer "F.Cu") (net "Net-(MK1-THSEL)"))
 (segment (start 138.649496 87.9) (end 138.63 87.9) (width 0.2) (layer "F.Cu") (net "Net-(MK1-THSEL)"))
 (segment (start 137.853316 88.676684) (end 137.847504 88.676684) (width 0.2) (layer "F.Cu") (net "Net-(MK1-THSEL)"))
 (via (at 137.847504 88.676684) (size 0.6) (drill 0.3) (layers "F.Cu" "B.Cu") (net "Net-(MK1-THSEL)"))
 (segment (start 141.19 93.5) (end 139.85 93.5) (width 0.2) (layer "B.Cu") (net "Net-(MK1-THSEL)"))
 (segment (start 137.847504 91.497504) (end 137.847504 88.676684) (width 0.2) (layer "B.Cu") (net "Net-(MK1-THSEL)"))
 (segment (start 139.85 93.5) (end 137.847504 91.497504) (width 0.2) (layer "B.Cu") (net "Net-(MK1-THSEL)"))
 (segment (start 139.149622 88.450378) (end 138.825 88.775) (width 0.2) (layer "F.Cu") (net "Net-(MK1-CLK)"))
 (segment (start 138.825 88.775) (end 138.825 89.4) (width 0.2) (layer "F.Cu") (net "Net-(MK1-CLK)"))
 (segment (start 139.149622 87.900001) (end 139.149622 88.450378) (width 0.2) (layer "F.Cu") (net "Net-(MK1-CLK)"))
 (via (at 138.825 89.4) (size 0.6) (drill 0.3) (layers "F.Cu" "B.Cu") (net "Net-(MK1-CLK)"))
 (segment (start 141.3775 91.483) (end 139.558 91.483) (width 0.2) (layer "B.Cu") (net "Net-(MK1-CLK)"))
 (segment (start 139.558 91.483) (end 138.825 90.75) (width 0.2) (layer "B.Cu") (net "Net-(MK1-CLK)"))
 (segment (start 138.825 90.75) (end 138.825 89.4) (width 0.2) (layer "B.Cu") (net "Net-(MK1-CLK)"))
 (segment (start 141.3781 91.475) (end 141.3811 91.478) (width 0.2) (layer "B.Cu") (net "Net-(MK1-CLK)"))
 (segment (start 139.649748 89.05264) (end 139.649748 87.9) (width 0.2) (layer "F.Cu") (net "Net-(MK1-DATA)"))
 (segment (start 139.922108 89.325) (end 139.649748 89.05264) (width 0.2) (layer "F.Cu") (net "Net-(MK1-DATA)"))
 (segment (start 139.925 89.325) (end 139.922108 89.325) (width 0.2) (layer "F.Cu") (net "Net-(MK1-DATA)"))
 (via (at 139.925 89.325) (size 0.6) (drill 0.3) (layers "F.Cu" "B.Cu") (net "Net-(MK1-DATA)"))
 (segment (start 139.925 89.325) (end 140.425 89.825) (width 0.2) (layer "B.Cu") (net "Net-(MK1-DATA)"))
 (segment (start 140.425 89.825) (end 142.2231 89.825) (width 0.2) (layer "B.Cu") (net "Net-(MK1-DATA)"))
 (segment (start 143.0525 90.6544) (end 143.0525 90.663) (width 0.2) (layer "B.Cu") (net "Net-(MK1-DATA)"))
 (segment (start 142.2231 89.825) (end 143.0525 90.6544) (width 0.2) (layer "B.Cu") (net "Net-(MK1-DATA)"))
 (segment (start 140.149874 88.453474) (end 140.6964 89) (width 0.2) (layer "F.Cu") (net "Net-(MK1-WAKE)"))
 (segment (start 140.149874 87.900001) (end 140.149874 88.453474) (width 0.2) (layer "F.Cu") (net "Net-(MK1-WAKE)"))
 (via (at 140.6964 89) (size 0.6) (drill 0.3) (layers "F.Cu" "B.Cu") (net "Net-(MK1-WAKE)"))
 (segment (start 143.132107 89) (end 144.4 90.267893) (width 0.2) (layer "B.Cu") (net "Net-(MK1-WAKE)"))
 (segment (start 140.6964 89) (end 143.132107 89) (width 0.2) (layer "B.Cu") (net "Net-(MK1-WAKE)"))
 (segment (start 144.4 90.267893) (end 144.4 92.3386) (width 0.2) (layer "B.Cu") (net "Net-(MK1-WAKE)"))
 (segment (start 143.24 93.4986) (end 143.24 93.5) (width 0.2) (layer "B.Cu") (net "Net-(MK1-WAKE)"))
 (segment (start 144.4 92.3386) (end 143.24 93.4986) (width 0.2) (layer "B.Cu") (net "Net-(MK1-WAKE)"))
 (segment (start 140.149874 85.079126) (end 140.149874 85.512399) (width 0.2) (layer "F.Cu") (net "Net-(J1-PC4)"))
 (segment (start 140.404 84.825) (end 140.149874 85.079126) (width 0.2) (layer "F.Cu") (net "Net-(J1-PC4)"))
 (segment (start 142.203948 86.053948) (end 140.975 84.825) (width 0.2) (layer "F.Cu") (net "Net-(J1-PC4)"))
 (segment (start 140.975 84.825) (end 140.404 84.825) (width 0.2) (layer "F.Cu") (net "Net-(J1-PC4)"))
 (segment (start 142.203948 86.891468) (end 142.203948 86.053948) (width 0.2) (layer "F.Cu") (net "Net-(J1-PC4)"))
 (via (at 142.203948 86.891468) (size 0.6) (drill 0.3) (layers "F.Cu" "B.Cu") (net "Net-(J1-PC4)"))
 (segment (start 142.020416 87.075) (end 140.825 87.075) (width 0.2) (layer "B.Cu") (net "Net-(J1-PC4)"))
 (segment (start 140.19 87.71) (end 140.19 88.18) (width 0.2) (layer "B.Cu") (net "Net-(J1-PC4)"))
 (segment (start 140.825 87.075) (end 140.19 87.71) (width 0.2) (layer "B.Cu") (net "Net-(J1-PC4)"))
 (segment (start 142.203948 86.891468) (end 142.020416 87.075) (width 0.2) (layer "B.Cu") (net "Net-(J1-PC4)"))
 (segment (start 140.225 84.35) (end 139.649748 84.925252) (width 0.2) (layer "F.Cu") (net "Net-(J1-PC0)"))
 (segment (start 142.65 84.35) (end 140.225 84.35) (width 0.2) (layer "F.Cu") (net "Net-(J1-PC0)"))
 (segment (start 143.575 85.275) (end 142.65 84.35) (width 0.2) (layer "F.Cu") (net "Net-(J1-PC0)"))
 (segment (start 143.575 85.45) (end 143.575 85.275) (width 0.2) (layer "F.Cu") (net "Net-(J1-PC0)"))
 (segment (start 139.649748 84.925252) (end 139.649748 85.5124) (width 0.2) (layer "F.Cu") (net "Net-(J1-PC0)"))
 (via (at 143.575 85.45) (size 0.6) (drill 0.3) (layers "F.Cu" "B.Cu") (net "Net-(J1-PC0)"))
 (segment (start 139.175 86.025) (end 143.305 86.025) (width 0.2) (layer "B.Cu") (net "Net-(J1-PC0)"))
 (segment (start 138.99 85.47) (end 138.99 85.84) (width 0.2) (layer "B.Cu") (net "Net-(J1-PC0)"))
 (segment (start 143.305 86.025) (end 143.575 85.755) (width 0.2) (layer "B.Cu") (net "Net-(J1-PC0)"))
 (segment (start 138.99 85.84) (end 139.175 86.025) (width 0.2) (layer "B.Cu") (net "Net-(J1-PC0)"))
 (segment (start 143.575 85.755) (end 143.575 85.45) (width 0.2) (layer "B.Cu") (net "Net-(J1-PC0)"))
 (segment (start 139.149622 85.079126) (end 139.149622 85.5124) (width 0.2) (layer "F.Cu") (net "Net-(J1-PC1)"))
 (segment (start 138.920496 84.85) (end 139.149622 85.079126) (width 0.2) (layer "F.Cu") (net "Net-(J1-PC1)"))
 (segment (start 138.028554 84.85) (end 138.920496 84.85) (width 0.2) (layer "F.Cu") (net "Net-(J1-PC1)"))
 (via (at 138.028554 84.85) (size 0.6) (drill 0.3) (layers "F.Cu" "B.Cu") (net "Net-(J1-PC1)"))
 (segment (start 138.028554 84.85) (end 137.675 84.85) (width 0.2) (layer "B.Cu") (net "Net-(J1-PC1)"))
 (segment (start 137.675 84.85) (end 137.11 85.415) (width 0.2) (layer "B.Cu") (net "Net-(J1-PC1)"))
 (segment (start 137.8 87.25) (end 138.53 87.25) (width 0.2) (layer "B.Cu") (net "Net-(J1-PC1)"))
 (segment (start 138.99 87.71) (end 138.99 88.18) (width 0.2) (layer "B.Cu") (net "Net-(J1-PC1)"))
 (segment (start 137.11 85.415) (end 137.11 86.56) (width 0.2) (layer "B.Cu") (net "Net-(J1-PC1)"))
 (segment (start 137.11 86.56) (end 137.8 87.25) (width 0.2) (layer "B.Cu") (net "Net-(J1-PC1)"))
 (segment (start 138.53 87.25) (end 138.99 87.71) (width 0.2) (layer "B.Cu") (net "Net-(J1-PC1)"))
 (segment (start 137.61 85.76) (end 137.61 85.91) (width 0.2) (layer "F.Cu") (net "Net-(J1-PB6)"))
 (segment (start 138.649496 85.5124) (end 137.8576 85.5124) (width 0.2) (layer "F.Cu") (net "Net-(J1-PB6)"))
 (segment (start 137.8576 85.5124) (end 137.61 85.76) (width 0.2) (layer "F.Cu") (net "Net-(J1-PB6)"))
 (via (at 137.61 85.91) (size 0.6) (drill 0.3) (layers "F.Cu" "B.Cu") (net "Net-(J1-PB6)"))
 (segment (start 141.990945 86.391468) (end 141.807413 86.575) (width 0.2) (layer "B.Cu") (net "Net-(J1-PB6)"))
 (segment (start 138.025 86.575) (end 137.61 86.16) (width 0.2) (layer "B.Cu") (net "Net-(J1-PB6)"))
 (segment (start 142.703948 86.684361) (end 142.411055 86.391468) (width 0.2) (layer "B.Cu") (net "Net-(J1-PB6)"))
 (segment (start 141.79 87.81) (end 142.208532 87.391468) (width 0.2) (layer "B.Cu") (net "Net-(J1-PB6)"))
 (segment (start 142.208532 87.391468) (end 142.411055 87.391468) (width 0.2) (layer "B.Cu") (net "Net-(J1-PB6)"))
 (segment (start 141.79 88.18) (end 141.79 87.81) (width 0.2) (layer "B.Cu") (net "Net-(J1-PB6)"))
 (segment (start 142.411055 87.391468) (end 142.703948 87.098575) (width 0.2) (layer "B.Cu") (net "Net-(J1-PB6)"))
 (segment (start 137.61 86.16) (end 137.61 85.91) (width 0.2) (layer "B.Cu") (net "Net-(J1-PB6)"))
 (segment (start 142.703948 87.098575) (end 142.703948 86.684361) (width 0.2) (layer "B.Cu") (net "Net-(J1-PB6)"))
 (segment (start 142.411055 86.391468) (end 141.990945 86.391468) (width 0.2) (layer "B.Cu") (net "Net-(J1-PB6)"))
 (segment (start 141.807413 86.575) (end 138.025 86.575) (width 0.2) (layer "B.Cu") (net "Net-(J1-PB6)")))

